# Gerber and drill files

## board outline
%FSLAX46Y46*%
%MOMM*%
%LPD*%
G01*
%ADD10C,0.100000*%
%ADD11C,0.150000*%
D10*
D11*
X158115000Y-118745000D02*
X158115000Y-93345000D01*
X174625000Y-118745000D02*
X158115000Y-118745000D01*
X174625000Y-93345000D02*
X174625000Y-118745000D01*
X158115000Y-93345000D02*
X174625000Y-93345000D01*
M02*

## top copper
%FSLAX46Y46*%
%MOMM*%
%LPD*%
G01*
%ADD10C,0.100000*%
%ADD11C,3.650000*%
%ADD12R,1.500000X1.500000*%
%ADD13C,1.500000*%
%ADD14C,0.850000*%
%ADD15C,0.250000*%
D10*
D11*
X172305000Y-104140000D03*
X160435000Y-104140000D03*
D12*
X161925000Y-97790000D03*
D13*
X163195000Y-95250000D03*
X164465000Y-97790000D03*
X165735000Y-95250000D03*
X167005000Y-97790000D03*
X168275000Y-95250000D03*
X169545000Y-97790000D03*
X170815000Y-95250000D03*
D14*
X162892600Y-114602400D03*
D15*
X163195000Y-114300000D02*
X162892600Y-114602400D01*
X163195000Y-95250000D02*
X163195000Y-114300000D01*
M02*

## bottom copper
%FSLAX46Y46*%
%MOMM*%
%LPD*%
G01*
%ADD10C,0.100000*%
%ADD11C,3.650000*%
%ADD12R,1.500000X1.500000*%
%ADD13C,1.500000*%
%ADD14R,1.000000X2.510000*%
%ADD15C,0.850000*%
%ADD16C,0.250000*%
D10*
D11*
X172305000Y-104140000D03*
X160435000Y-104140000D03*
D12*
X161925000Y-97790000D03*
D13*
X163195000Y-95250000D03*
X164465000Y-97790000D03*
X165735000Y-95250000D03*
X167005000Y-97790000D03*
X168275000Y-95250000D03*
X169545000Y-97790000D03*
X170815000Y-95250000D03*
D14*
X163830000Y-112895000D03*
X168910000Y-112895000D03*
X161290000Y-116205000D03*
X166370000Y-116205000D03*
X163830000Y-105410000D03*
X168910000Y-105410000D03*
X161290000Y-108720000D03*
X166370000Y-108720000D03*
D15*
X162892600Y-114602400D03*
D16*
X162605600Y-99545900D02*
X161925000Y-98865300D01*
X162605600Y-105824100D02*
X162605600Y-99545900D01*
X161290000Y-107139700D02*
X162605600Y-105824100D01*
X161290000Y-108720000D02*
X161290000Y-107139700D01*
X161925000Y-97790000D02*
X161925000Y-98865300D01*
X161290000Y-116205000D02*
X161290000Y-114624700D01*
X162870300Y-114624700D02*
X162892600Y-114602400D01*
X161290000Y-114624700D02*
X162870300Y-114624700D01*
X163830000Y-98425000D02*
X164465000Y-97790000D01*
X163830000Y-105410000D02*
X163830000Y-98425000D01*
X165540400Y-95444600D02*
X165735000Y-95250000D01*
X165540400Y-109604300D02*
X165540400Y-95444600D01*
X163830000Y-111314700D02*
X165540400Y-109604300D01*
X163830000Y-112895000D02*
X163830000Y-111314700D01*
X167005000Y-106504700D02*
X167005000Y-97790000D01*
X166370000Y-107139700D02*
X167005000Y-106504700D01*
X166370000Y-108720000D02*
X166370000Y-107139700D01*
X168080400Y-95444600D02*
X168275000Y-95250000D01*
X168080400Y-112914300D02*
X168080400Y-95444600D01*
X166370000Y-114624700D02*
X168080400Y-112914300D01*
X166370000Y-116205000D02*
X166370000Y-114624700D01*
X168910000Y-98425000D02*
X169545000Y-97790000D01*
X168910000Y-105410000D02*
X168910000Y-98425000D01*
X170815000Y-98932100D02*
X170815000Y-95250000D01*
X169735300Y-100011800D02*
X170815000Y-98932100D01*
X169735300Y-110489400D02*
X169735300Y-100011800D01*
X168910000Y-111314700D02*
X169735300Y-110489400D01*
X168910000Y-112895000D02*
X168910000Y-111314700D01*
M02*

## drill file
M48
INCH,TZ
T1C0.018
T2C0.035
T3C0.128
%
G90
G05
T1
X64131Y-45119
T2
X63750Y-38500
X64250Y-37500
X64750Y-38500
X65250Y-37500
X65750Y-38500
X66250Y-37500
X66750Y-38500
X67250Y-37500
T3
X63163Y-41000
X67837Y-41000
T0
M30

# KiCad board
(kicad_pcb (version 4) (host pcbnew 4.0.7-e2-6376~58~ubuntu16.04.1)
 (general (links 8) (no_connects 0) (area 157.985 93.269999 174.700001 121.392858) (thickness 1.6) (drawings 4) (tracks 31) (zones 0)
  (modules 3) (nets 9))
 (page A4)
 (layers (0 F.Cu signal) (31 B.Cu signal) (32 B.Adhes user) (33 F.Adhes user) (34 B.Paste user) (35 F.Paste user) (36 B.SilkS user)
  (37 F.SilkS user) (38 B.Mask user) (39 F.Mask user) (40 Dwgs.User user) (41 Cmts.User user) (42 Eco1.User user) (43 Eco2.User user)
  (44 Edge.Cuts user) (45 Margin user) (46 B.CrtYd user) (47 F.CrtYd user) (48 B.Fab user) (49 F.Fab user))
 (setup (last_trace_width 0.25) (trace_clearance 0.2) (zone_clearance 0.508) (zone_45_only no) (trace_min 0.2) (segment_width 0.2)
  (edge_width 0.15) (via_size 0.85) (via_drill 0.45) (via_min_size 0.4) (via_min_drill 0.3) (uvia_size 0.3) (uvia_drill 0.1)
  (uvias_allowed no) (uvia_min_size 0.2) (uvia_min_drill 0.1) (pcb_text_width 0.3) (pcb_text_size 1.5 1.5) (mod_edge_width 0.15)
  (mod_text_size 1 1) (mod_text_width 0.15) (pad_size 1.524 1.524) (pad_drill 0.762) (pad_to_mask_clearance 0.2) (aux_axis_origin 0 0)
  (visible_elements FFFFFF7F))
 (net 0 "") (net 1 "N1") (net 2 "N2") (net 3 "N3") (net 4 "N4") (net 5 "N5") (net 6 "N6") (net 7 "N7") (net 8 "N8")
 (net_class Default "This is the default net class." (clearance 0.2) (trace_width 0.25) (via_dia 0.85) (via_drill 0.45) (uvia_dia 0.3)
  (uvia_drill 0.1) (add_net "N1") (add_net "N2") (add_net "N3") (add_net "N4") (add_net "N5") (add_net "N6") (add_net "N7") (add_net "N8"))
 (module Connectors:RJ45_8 (layer F.Cu) (at 161.925 97.79)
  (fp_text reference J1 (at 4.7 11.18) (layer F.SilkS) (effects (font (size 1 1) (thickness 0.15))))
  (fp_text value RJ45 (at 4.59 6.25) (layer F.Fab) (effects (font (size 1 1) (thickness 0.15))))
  (pad Hole np_thru_hole circle (at 10.38 6.35) (size 3.65 3.65) (drill 3.25) (layers *.Cu *.SilkS *.Mask))
  (pad Hole np_thru_hole circle (at -1.49 6.35) (size 3.65 3.65) (drill 3.25) (layers *.Cu *.SilkS *.Mask))
  (pad 1 thru_hole rect (at 0 0) (size 1.5 1.5) (drill 0.9) (layers *.Cu *.Mask) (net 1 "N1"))
  (pad 2 thru_hole circle (at 1.27 -2.54) (size 1.5 1.5) (drill 0.9) (layers *.Cu *.Mask) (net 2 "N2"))
  (pad 3 thru_hole circle (at 2.54 0) (size 1.5 1.5) (drill 0.9) (layers *.Cu *.Mask) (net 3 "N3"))
  (pad 4 thru_hole circle (at 3.81 -2.54) (size 1.5 1.5) (drill 0.9) (layers *.Cu *.Mask) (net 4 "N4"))
  (pad 5 thru_hole circle (at 5.08 0) (size 1.5 1.5) (drill 0.9) (layers *.Cu *.Mask) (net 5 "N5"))
  (pad 6 thru_hole circle (at 6.35 -2.54) (size 1.5 1.5) (drill 0.9) (layers *.Cu *.Mask) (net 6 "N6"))
  (pad 7 thru_hole circle (at 7.62 0) (size 1.5 1.5) (drill 0.9) (layers *.Cu *.Mask) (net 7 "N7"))
  (pad 8 thru_hole circle (at 8.89 -2.54) (size 1.5 1.5) (drill 0.9) (layers *.Cu *.Mask) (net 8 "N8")))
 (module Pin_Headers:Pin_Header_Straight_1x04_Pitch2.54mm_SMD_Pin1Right (layer B.Cu) (at 165.1 114.55 270)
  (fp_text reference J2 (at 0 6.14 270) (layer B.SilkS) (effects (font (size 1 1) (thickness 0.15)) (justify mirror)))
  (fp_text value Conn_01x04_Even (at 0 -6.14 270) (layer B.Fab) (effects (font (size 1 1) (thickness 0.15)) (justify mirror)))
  (pad 2 smd rect (at -1.655 1.27 270) (size 2.51 1) (layers B.Cu B.Paste B.Mask) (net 4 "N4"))
  (pad 4 smd rect (at -1.655 -3.81 270) (size 2.51 1) (layers B.Cu B.Paste B.Mask) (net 8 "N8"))
  (pad 1 smd rect (at 1.655 3.81 270) (size 2.51 1) (layers B.Cu B.Paste B.Mask) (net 2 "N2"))
  (pad 3 smd rect (at 1.655 -1.27 270) (size 2.51 1) (layers B.Cu B.Paste B.Mask) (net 6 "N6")))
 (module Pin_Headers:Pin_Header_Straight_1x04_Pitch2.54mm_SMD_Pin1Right (layer B.Cu) (at 165.1 107.065 270)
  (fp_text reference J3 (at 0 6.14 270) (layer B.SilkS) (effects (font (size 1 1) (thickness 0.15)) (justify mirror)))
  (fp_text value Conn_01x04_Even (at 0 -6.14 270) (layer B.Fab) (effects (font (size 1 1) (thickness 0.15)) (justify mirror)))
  (pad 2 smd rect (at -1.655 1.27 270) (size 2.51 1) (layers B.Cu B.Paste B.Mask) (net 3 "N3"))
  (pad 4 smd rect (at -1.655 -3.81 270) (size 2.51 1) (layers B.Cu B.Paste B.Mask) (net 7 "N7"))
  (pad 1 smd rect (at 1.655 3.81 270) (size 2.51 1) (layers B.Cu B.Paste B.Mask) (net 1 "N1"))
  (pad 3 smd rect (at 1.655 -1.27 270) (size 2.51 1) (layers B.Cu B.Paste B.Mask) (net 5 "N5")))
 (gr_line (start 158.115 118.745) (end 158.115 93.345) (layer Edge.Cuts) (width 0.15))
 (gr_line (start 174.625 118.745) (end 158.115 118.745) (layer Edge.Cuts) (width 0.15))
 (gr_line (start 174.625 93.345) (end 174.625 118.745) (layer Edge.Cuts) (width 0.15))
 (gr_line (start 158.115 93.345) (end 174.625 93.345) (layer Edge.Cuts) (width 0.15))
 (segment (start 162.6056 99.5459) (end 161.925 98.8653) (width 0.25) (layer B.Cu) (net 1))
 (segment (start 162.6056 105.8241) (end 162.6056 99.5459) (width 0.25) (layer B.Cu) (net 1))
 (segment (start 161.29 107.1397) (end 162.6056 105.8241) (width 0.25) (layer B.Cu) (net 1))
 (segment (start 161.29 108.72) (end 161.29 107.1397) (width 0.25) (layer B.Cu) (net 1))
 (segment (start 161.925 97.79) (end 161.925 98.8653) (width 0.25) (layer B.Cu) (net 1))
 (via (at 162.8926 114.6024) (size 0.85) (layers F.Cu B.Cu) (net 2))
 (segment (start 161.29 116.205) (end 161.29 114.6247) (width 0.25) (layer B.Cu) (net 2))
 (segment (start 162.8703 114.6247) (end 162.8926 114.6024) (width 0.25) (layer B.Cu) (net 2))
 (segment (start 161.29 114.6247) (end 162.8703 114.6247) (width 0.25) (layer B.Cu) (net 2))
 (segment (start 163.195 114.3) (end 162.8926 114.6024) (width 0.25) (layer F.Cu) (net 2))
 (segment (start 163.195 95.25) (end 163.195 114.3) (width 0.25) (layer F.Cu) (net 2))
 (segment (start 163.83 98.425) (end 164.465 97.79) (width 0.25) (layer B.Cu) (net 3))
 (segment (start 163.83 105.41) (end 163.83 98.425) (width 0.25) (layer B.Cu) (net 3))
 (segment (start 165.5404 95.4446) (end 165.735 95.25) (width 0.25) (layer B.Cu) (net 4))
 (segment (start 165.5404 109.6043) (end 165.5404 95.4446) (width 0.25) (layer B.Cu) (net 4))
 (segment (start 163.83 111.3147) (end 165.5404 109.6043) (width 0.25) (layer B.Cu) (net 4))
 (segment (start 163.83 112.895) (end 163.83 111.3147) (width 0.25) (layer B.Cu) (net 4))
 (segment (start 167.005 106.5047) (end 167.005 97.79) (width 0.25) (layer B.Cu) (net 5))
 (segment (start 166.37 107.1397) (end 167.005 106.5047) (width 0.25) (layer B.Cu) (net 5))
 (segment (start 166.37 108.72) (end 166.37 107.1397) (width 0.25) (layer B.Cu) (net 5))
 (segment (start 168.0804 95.4446) (end 168.275 95.25) (width 0.25) (layer B.Cu) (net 6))
 (segment (start 168.0804 112.9143) (end 168.0804 95.4446) (width 0.25) (layer B.Cu) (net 6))
 (segment (start 166.37 114.6247) (end 168.0804 112.9143) (width 0.25) (layer B.Cu) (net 6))
 (segment (start 166.37 116.205) (end 166.37 114.6247) (width 0.25) (layer B.Cu) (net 6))
 (segment (start 168.91 98.425) (end 169.545 97.79) (width 0.25) (layer B.Cu) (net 7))
 (segment (start 168.91 105.41) (end 168.91 98.425) (width 0.25) (layer B.Cu) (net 7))
 (segment (start 170.815 98.9321) (end 170.815 95.25) (width 0.25) (layer B.Cu) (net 8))
 (segment (start 169.7353 100.0118) (end 170.815 98.9321) (width 0.25) (layer B.Cu) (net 8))
 (segment (start 169.7353 110.4894) (end 169.7353 100.0118) (width 0.25) (layer B.Cu) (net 8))
 (segment (start 168.91 111.3147) (end 169.7353 110.4894) (width 0.25) (layer B.Cu) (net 8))
 (segment (start 168.91 112.895) (end 168.91 111.3147) (width 0.25) (layer B.Cu) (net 8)))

